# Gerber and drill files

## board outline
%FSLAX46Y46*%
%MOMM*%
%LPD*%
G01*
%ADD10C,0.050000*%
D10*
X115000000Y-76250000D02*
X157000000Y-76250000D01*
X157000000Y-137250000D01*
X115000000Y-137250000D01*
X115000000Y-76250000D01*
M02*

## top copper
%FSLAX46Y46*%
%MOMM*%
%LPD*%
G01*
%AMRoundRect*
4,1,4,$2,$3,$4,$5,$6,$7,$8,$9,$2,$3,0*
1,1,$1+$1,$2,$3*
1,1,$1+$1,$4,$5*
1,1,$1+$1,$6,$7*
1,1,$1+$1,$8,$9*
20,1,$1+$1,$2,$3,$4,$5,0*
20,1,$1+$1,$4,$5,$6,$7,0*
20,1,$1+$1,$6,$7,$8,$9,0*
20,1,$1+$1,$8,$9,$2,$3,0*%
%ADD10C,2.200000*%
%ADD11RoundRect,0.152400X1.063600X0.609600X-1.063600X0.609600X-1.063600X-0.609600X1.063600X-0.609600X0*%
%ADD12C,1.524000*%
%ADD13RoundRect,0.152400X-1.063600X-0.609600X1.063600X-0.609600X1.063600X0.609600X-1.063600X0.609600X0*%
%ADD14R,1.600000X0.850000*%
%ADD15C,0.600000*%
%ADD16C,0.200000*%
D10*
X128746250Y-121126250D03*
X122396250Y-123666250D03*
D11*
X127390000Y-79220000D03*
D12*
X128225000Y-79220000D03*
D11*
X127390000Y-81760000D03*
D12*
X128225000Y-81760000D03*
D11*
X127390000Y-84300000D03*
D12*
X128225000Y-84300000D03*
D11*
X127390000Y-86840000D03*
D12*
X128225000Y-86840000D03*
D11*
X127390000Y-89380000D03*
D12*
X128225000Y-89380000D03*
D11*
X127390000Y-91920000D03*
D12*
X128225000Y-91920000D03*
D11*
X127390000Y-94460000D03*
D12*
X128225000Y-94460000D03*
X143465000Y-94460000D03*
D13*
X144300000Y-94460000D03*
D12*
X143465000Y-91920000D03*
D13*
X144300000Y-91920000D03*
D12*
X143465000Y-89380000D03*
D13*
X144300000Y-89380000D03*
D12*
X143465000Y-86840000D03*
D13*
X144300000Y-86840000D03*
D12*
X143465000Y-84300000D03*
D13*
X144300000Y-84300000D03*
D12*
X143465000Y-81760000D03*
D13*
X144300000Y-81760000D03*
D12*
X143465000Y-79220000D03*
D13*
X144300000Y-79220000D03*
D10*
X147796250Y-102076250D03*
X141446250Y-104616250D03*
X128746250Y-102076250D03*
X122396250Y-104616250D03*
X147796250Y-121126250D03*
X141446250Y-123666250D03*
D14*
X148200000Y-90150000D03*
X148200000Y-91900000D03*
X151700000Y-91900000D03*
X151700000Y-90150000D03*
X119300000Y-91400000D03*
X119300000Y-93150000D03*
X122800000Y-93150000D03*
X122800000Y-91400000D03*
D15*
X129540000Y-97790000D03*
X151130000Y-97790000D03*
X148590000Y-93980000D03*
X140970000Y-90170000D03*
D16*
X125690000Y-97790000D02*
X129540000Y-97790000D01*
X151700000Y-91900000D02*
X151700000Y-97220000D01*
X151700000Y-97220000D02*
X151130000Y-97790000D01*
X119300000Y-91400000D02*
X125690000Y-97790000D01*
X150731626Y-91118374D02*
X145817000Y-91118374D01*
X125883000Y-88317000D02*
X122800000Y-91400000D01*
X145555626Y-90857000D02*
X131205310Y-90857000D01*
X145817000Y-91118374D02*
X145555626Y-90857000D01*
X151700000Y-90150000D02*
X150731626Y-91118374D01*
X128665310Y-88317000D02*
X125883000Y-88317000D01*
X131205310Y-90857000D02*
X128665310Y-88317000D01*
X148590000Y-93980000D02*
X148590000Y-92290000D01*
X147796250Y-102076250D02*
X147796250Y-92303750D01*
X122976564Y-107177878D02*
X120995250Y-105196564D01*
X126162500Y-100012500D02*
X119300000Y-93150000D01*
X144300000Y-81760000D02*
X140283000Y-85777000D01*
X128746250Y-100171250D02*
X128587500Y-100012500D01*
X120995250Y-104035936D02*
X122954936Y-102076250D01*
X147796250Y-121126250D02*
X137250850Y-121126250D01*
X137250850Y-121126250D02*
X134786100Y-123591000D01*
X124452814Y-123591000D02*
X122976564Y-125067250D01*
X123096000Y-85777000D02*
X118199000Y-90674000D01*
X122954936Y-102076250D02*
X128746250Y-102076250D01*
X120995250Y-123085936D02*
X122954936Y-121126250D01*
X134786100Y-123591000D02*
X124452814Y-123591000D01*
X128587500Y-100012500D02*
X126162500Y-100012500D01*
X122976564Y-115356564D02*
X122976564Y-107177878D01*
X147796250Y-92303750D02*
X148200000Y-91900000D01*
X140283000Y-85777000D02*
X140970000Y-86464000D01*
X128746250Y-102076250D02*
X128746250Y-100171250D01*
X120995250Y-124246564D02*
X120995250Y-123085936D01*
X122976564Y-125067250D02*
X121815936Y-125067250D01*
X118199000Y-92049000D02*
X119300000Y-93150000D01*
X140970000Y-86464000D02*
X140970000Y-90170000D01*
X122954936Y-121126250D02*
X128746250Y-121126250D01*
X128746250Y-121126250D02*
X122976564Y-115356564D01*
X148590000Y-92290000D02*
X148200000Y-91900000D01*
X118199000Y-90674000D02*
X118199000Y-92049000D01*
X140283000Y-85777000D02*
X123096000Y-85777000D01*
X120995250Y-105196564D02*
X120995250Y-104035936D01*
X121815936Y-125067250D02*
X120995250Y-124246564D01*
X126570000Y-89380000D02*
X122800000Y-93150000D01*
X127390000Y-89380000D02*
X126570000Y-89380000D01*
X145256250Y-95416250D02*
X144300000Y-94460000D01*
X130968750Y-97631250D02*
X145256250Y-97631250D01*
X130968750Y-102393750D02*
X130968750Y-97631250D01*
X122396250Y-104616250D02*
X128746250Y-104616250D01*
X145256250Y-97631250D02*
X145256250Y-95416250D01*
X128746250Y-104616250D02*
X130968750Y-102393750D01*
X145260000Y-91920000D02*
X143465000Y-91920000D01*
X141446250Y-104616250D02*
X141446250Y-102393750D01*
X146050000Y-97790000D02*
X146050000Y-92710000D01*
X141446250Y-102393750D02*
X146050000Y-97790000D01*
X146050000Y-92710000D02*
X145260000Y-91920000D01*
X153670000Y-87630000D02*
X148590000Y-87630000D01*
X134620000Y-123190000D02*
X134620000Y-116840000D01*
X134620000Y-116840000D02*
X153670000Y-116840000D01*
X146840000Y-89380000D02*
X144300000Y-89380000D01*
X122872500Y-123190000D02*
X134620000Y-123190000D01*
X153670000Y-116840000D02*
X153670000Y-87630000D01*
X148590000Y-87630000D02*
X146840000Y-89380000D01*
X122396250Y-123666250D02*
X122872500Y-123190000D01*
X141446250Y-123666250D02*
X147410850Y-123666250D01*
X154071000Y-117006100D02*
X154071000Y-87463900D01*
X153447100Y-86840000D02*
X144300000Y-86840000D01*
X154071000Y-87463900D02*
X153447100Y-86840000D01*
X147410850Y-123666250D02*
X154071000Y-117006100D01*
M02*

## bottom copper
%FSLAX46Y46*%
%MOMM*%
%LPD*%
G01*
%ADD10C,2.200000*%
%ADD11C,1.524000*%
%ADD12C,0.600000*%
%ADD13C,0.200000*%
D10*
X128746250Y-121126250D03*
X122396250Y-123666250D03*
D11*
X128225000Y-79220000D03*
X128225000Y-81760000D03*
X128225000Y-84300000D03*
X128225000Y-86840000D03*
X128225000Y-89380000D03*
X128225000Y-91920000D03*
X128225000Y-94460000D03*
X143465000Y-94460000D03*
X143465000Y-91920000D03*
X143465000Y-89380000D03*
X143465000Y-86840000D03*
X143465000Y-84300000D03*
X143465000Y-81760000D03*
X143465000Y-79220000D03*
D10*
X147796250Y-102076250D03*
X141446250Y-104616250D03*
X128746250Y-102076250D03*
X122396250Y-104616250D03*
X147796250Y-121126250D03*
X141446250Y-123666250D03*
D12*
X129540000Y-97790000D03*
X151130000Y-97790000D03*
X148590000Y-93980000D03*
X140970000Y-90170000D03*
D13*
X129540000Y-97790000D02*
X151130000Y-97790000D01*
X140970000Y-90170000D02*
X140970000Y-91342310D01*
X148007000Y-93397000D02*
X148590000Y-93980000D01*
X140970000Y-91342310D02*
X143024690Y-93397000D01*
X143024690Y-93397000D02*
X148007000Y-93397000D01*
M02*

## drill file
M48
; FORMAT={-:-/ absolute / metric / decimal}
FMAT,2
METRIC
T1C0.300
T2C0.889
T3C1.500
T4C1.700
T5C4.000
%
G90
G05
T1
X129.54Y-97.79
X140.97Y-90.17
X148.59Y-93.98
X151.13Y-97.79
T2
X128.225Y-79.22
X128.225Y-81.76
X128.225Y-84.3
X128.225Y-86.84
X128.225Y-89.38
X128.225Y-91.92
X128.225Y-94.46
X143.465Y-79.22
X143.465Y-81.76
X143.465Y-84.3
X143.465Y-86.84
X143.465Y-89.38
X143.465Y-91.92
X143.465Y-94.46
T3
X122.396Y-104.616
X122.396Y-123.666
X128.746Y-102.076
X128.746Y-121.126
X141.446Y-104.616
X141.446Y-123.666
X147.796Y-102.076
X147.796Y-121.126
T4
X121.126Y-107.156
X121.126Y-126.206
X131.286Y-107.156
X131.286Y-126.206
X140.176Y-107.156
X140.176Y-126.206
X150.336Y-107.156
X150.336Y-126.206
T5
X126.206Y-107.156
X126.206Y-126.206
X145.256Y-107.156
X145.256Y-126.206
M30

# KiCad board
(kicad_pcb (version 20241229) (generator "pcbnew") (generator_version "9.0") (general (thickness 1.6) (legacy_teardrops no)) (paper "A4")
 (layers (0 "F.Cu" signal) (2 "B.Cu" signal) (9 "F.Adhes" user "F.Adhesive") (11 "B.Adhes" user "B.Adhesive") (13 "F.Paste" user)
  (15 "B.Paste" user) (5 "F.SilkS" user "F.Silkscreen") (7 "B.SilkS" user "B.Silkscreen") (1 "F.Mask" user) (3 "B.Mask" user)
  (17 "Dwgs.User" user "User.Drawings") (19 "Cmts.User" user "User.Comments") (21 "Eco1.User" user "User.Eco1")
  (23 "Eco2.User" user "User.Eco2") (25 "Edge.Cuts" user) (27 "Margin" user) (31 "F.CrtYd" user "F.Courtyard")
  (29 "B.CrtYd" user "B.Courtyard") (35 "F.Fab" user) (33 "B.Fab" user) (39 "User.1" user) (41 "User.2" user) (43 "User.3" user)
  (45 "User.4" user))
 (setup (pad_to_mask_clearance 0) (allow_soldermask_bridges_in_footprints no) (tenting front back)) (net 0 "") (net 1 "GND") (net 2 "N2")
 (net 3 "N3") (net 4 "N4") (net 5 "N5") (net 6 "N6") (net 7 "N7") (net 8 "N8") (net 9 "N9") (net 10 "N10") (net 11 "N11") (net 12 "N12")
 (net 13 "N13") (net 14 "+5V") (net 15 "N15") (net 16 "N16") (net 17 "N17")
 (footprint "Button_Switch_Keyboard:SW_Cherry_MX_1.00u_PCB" (layer "F.Cu") (at 128.74625 121.12625)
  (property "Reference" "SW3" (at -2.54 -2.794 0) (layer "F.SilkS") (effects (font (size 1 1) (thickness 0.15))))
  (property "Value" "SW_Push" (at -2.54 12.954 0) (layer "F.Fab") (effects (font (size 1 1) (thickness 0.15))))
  (pad "" np_thru_hole circle (at -7.62 5.08) (size 1.7 1.7) (drill 1.7) (layers "*.Cu" "*.Mask"))
  (pad "" np_thru_hole circle (at -2.54 5.08) (size 4 4) (drill 4) (layers "*.Cu" "*.Mask"))
  (pad "" np_thru_hole circle (at 2.54 5.08) (size 1.7 1.7) (drill 1.7) (layers "*.Cu" "*.Mask"))
  (pad "1" thru_hole circle (at 0 0) (size 2.2 2.2) (drill 1.5) (layers "*.Cu" "*.Mask") (remove_unused_layers no) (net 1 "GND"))
  (pad "2" thru_hole circle (at -6.35 2.54) (size 2.2 2.2) (drill 1.5) (layers "*.Cu" "*.Mask") (remove_unused_layers no) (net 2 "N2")))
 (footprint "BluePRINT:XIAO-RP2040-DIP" (layer "F.Cu") (at 135.845 86.84)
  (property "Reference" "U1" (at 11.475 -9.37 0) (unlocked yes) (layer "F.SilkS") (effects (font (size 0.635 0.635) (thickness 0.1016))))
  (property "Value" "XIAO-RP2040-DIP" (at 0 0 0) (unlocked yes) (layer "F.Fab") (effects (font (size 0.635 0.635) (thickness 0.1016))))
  (pad "1" smd roundrect (at -8.455 -7.62 180) (size 2.432 1.524) (layers "F.Cu" "F.Mask") (roundrect_rratio 0.1) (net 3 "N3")
   (thermal_bridge_angle 45))
  (pad "1" thru_hole circle (at -7.62 -7.62 180) (size 1.524 1.524) (drill 0.889) (layers "*.Cu" "*.Mask") (remove_unused_layers no)
   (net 3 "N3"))
  (pad "2" smd roundrect (at -8.455 -5.08 180) (size 2.432 1.524) (layers "F.Cu" "F.Mask") (roundrect_rratio 0.1) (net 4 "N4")
   (thermal_bridge_angle 45))
  (pad "2" thru_hole circle (at -7.62 -5.08 180) (size 1.524 1.524) (drill 0.889) (layers "*.Cu" "*.Mask") (remove_unused_layers no)
   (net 4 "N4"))
  (pad "3" smd roundrect (at -8.455 -2.54 180) (size 2.432 1.524) (layers "F.Cu" "F.Mask") (roundrect_rratio 0.1) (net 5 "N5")
   (thermal_bridge_angle 45))
  (pad "3" thru_hole circle (at -7.62 -2.54 180) (size 1.524 1.524) (drill 0.889) (layers "*.Cu" "*.Mask") (remove_unused_layers no)
   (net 5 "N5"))
  (pad "4" smd roundrect (at -8.455 0 180) (size 2.432 1.524) (layers "F.Cu" "F.Mask") (roundrect_rratio 0.1) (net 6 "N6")
   (thermal_bridge_angle 45))
  (pad "4" thru_hole circle (at -7.62 0 180) (size 1.524 1.524) (drill 0.889) (layers "*.Cu" "*.Mask") (remove_unused_layers no)
   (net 6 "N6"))
  (pad "5" smd roundrect (at -8.455 2.54 180) (size 2.432 1.524) (layers "F.Cu" "F.Mask") (roundrect_rratio 0.1) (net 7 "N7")
   (thermal_bridge_angle 45))
  (pad "5" thru_hole circle (at -7.62 2.54 180) (size 1.524 1.524) (drill 0.889) (layers "*.Cu" "*.Mask") (remove_unused_layers no)
   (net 7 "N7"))
  (pad "6" smd roundrect (at -8.455 5.08 180) (size 2.432 1.524) (layers "F.Cu" "F.Mask") (roundrect_rratio 0.1) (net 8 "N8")
   (thermal_bridge_angle 45))
  (pad "6" thru_hole circle (at -7.62 5.08 180) (size 1.524 1.524) (drill 0.889) (layers "*.Cu" "*.Mask") (remove_unused_layers no)
   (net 8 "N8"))
  (pad "7" smd roundrect (at -8.455 7.62 180) (size 2.432 1.524) (layers "F.Cu" "F.Mask") (roundrect_rratio 0.1) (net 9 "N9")
   (thermal_bridge_angle 45))
  (pad "7" thru_hole circle (at -7.62 7.62 180) (size 1.524 1.524) (drill 0.889) (layers "*.Cu" "*.Mask") (remove_unused_layers no)
   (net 9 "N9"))
  (pad "8" thru_hole circle (at 7.62 7.62) (size 1.524 1.524) (drill 0.889) (layers "*.Cu" "*.Mask") (remove_unused_layers no)
   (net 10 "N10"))
  (pad "8" smd roundrect (at 8.455 7.62) (size 2.432 1.524) (layers "F.Cu" "F.Mask") (roundrect_rratio 0.1) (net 10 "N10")
   (thermal_bridge_angle 45))
  (pad "9" thru_hole circle (at 7.62 5.08) (size 1.524 1.524) (drill 0.889) (layers "*.Cu" "*.Mask") (remove_unused_layers no)
   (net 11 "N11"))
  (pad "9" smd roundrect (at 8.455 5.08) (size 2.432 1.524) (layers "F.Cu" "F.Mask") (roundrect_rratio 0.1) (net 11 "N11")
   (thermal_bridge_angle 45))
  (pad "10" thru_hole circle (at 7.62 2.54) (size 1.524 1.524) (drill 0.889) (layers "*.Cu" "*.Mask") (remove_unused_layers no) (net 2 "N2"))
  (pad "10" smd roundrect (at 8.455 2.54) (size 2.432 1.524) (layers "F.Cu" "F.Mask") (roundrect_rratio 0.1) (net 2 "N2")
   (thermal_bridge_angle 45))
  (pad "11" thru_hole circle (at 7.62 0) (size 1.524 1.524) (drill 0.889) (layers "*.Cu" "*.Mask") (remove_unused_layers no) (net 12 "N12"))
  (pad "11" smd roundrect (at 8.455 0) (size 2.432 1.524) (layers "F.Cu" "F.Mask") (roundrect_rratio 0.1) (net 12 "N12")
   (thermal_bridge_angle 45))
  (pad "12" thru_hole circle (at 7.62 -2.54) (size 1.524 1.524) (drill 0.889) (layers "*.Cu" "*.Mask") (remove_unused_layers no)
   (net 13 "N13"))
  (pad "12" smd roundrect (at 8.455 -2.54) (size 2.432 1.524) (layers "F.Cu" "F.Mask") (roundrect_rratio 0.1) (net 13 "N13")
   (thermal_bridge_angle 45))
  (pad "13" thru_hole circle (at 7.62 -5.08) (size 1.524 1.524) (drill 0.889) (layers "*.Cu" "*.Mask") (remove_unused_layers no)
   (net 1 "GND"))
  (pad "13" smd roundrect (at 8.455 -5.08) (size 2.432 1.524) (layers "F.Cu" "F.Mask") (roundrect_rratio 0.1) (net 1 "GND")
   (thermal_bridge_angle 45))
  (pad "14" thru_hole circle (at 7.62 -7.62) (size 1.524 1.524) (drill 0.889) (layers "*.Cu" "*.Mask") (remove_unused_layers no)
   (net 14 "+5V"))
  (pad "14" smd roundrect (at 8.455 -7.62) (size 2.432 1.524) (layers "F.Cu" "F.Mask") (roundrect_rratio 0.1) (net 14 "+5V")
   (thermal_bridge_angle 45)))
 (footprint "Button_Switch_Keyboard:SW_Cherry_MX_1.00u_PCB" (layer "F.Cu") (at 147.79625 102.07625)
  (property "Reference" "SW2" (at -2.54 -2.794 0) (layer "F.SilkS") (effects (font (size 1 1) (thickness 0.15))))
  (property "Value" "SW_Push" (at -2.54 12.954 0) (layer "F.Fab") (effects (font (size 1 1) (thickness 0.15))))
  (pad "" np_thru_hole circle (at -7.62 5.08) (size 1.7 1.7) (drill 1.7) (layers "*.Cu" "*.Mask"))
  (pad "" np_thru_hole circle (at -2.54 5.08) (size 4 4) (drill 4) (layers "*.Cu" "*.Mask"))
  (pad "" np_thru_hole circle (at 2.54 5.08) (size 1.7 1.7) (drill 1.7) (layers "*.Cu" "*.Mask"))
  (pad "1" thru_hole circle (at 0 0) (size 2.2 2.2) (drill 1.5) (layers "*.Cu" "*.Mask") (remove_unused_layers no) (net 1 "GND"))
  (pad "2" thru_hole circle (at -6.35 2.54) (size 2.2 2.2) (drill 1.5) (layers "*.Cu" "*.Mask") (remove_unused_layers no) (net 11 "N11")))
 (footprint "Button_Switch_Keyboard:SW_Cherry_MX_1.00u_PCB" (layer "F.Cu") (at 128.74625 102.07625)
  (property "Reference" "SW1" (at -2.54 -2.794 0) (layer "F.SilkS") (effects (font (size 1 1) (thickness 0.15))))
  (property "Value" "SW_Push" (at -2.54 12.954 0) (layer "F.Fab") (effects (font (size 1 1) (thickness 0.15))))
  (pad "" np_thru_hole circle (at -7.62 5.08) (size 1.7 1.7) (drill 1.7) (layers "*.Cu" "*.Mask"))
  (pad "" np_thru_hole circle (at -2.54 5.08) (size 4 4) (drill 4) (layers "*.Cu" "*.Mask"))
  (pad "" np_thru_hole circle (at 2.54 5.08) (size 1.7 1.7) (drill 1.7) (layers "*.Cu" "*.Mask"))
  (pad "1" thru_hole circle (at 0 0) (size 2.2 2.2) (drill 1.5) (layers "*.Cu" "*.Mask") (remove_unused_layers no) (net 1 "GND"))
  (pad "2" thru_hole circle (at -6.35 2.54) (size 2.2 2.2) (drill 1.5) (layers "*.Cu" "*.Mask") (remove_unused_layers no) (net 10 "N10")))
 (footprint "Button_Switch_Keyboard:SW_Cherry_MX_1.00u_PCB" (layer "F.Cu") (at 147.79625 121.12625)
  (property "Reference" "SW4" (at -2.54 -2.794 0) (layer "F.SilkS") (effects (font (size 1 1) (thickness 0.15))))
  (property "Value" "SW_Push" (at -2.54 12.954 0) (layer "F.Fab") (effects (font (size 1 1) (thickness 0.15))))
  (pad "" np_thru_hole circle (at -7.62 5.08) (size 1.7 1.7) (drill 1.7) (layers "*.Cu" "*.Mask"))
  (pad "" np_thru_hole circle (at -2.54 5.08) (size 4 4) (drill 4) (layers "*.Cu" "*.Mask"))
  (pad "" np_thru_hole circle (at 2.54 5.08) (size 1.7 1.7) (drill 1.7) (layers "*.Cu" "*.Mask"))
  (pad "1" thru_hole circle (at 0 0) (size 2.2 2.2) (drill 1.5) (layers "*.Cu" "*.Mask") (remove_unused_layers no) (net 1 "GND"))
  (pad "2" thru_hole circle (at -6.35 2.54) (size 2.2 2.2) (drill 1.5) (layers "*.Cu" "*.Mask") (remove_unused_layers no) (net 12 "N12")))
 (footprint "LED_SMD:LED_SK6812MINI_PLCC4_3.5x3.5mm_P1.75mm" (layer "F.Cu") (at 149.95 91.025)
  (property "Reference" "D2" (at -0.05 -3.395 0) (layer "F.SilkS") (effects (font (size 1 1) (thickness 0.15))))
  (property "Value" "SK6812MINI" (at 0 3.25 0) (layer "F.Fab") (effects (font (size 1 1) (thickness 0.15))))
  (pad "1" smd rect (at -1.75 -0.875) (size 1.6 0.85) (layers "F.Cu" "F.Mask" "F.Paste") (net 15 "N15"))
  (pad "2" smd rect (at -1.75 0.875) (size 1.6 0.85) (layers "F.Cu" "F.Mask" "F.Paste") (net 1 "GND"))
  (pad "3" smd rect (at 1.75 0.875) (size 1.6 0.85) (layers "F.Cu" "F.Mask" "F.Paste") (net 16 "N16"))
  (pad "4" smd rect (at 1.75 -0.875) (size 1.6 0.85) (layers "F.Cu" "F.Mask" "F.Paste") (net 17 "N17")))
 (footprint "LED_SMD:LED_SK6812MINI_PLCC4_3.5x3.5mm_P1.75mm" (layer "F.Cu") (at 121.05 92.275)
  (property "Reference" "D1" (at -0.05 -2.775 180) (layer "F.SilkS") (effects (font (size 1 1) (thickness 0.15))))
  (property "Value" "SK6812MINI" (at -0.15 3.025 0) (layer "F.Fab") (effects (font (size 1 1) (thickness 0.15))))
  (pad "1" smd rect (at -1.75 -0.875) (size 1.6 0.85) (layers "F.Cu" "F.Mask" "F.Paste") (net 16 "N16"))
  (pad "2" smd rect (at -1.75 0.875) (size 1.6 0.85) (layers "F.Cu" "F.Mask" "F.Paste") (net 1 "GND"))
  (pad "3" smd rect (at 1.75 0.875) (size 1.6 0.85) (layers "F.Cu" "F.Mask" "F.Paste") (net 7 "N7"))
  (pad "4" smd rect (at 1.75 -0.875) (size 1.6 0.85) (layers "F.Cu" "F.Mask" "F.Paste") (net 17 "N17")))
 (gr_rect (start 115 76.25) (end 157 137.25) (stroke (width 0.05) (type default)) (fill no) (layer "Edge.Cuts"))
 (segment (start 125.69 97.79) (end 129.54 97.79) (width 0.2) (layer "F.Cu") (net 16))
 (segment (start 151.7 91.9) (end 151.7 97.22) (width 0.2) (layer "F.Cu") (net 16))
 (segment (start 151.7 97.22) (end 151.13 97.79) (width 0.2) (layer "F.Cu") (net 16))
 (segment (start 119.3 91.4) (end 125.69 97.79) (width 0.2) (layer "F.Cu") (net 16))
 (via (at 129.54 97.79) (size 0.6) (drill 0.3) (layers "F.Cu" "B.Cu") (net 16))
 (via (at 151.13 97.79) (size 0.6) (drill 0.3) (layers "F.Cu" "B.Cu") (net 16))
 (segment (start 129.54 97.79) (end 151.13 97.79) (width 0.2) (layer "B.Cu") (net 16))
 (segment (start 150.731626 91.118374) (end 145.817 91.118374) (width 0.2) (layer "F.Cu") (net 17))
 (segment (start 125.883 88.317) (end 122.8 91.4) (width 0.2) (layer "F.Cu") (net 17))
 (segment (start 145.555626 90.857) (end 131.20531 90.857) (width 0.2) (layer "F.Cu") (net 17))
 (segment (start 145.817 91.118374) (end 145.555626 90.857) (width 0.2) (layer "F.Cu") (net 17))
 (segment (start 151.7 90.15) (end 150.731626 91.118374) (width 0.2) (layer "F.Cu") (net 17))
 (segment (start 128.66531 88.317) (end 125.883 88.317) (width 0.2) (layer "F.Cu") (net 17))
 (segment (start 131.20531 90.857) (end 128.66531 88.317) (width 0.2) (layer "F.Cu") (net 17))
 (segment (start 148.59 93.98) (end 148.59 92.29) (width 0.2) (layer "F.Cu") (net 1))
 (segment (start 147.79625 102.07625) (end 147.79625 92.30375) (width 0.2) (layer "F.Cu") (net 1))
 (segment (start 122.976564 107.177878) (end 120.99525 105.196564) (width 0.2) (layer "F.Cu") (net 1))
 (segment (start 126.1625 100.0125) (end 119.3 93.15) (width 0.2) (layer "F.Cu") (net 1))
 (segment (start 144.3 81.76) (end 140.283 85.777) (width 0.2) (layer "F.Cu") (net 1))
 (segment (start 128.74625 100.17125) (end 128.5875 100.0125) (width 0.2) (layer "F.Cu") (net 1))
 (segment (start 120.99525 104.035936) (end 122.954936 102.07625) (width 0.2) (layer "F.Cu") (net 1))
 (segment (start 147.79625 121.12625) (end 137.25085 121.12625) (width 0.2) (layer "F.Cu") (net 1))
 (segment (start 137.25085 121.12625) (end 134.7861 123.591) (width 0.2) (layer "F.Cu") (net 1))
 (segment (start 124.452814 123.591) (end 122.976564 125.06725) (width 0.2) (layer "F.Cu") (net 1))
 (segment (start 123.096 85.777) (end 118.199 90.674) (width 0.2) (layer "F.Cu") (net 1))
 (segment (start 122.954936 102.07625) (end 128.74625 102.07625) (width 0.2) (layer "F.Cu") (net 1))
 (segment (start 120.99525 123.085936) (end 122.954936 121.12625) (width 0.2) (layer "F.Cu") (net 1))
 (segment (start 134.7861 123.591) (end 124.452814 123.591) (width 0.2) (layer "F.Cu") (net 1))
 (segment (start 128.5875 100.0125) (end 126.1625 100.0125) (width 0.2) (layer "F.Cu") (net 1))
 (segment (start 122.976564 115.356564) (end 122.976564 107.177878) (width 0.2) (layer "F.Cu") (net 1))
 (segment (start 147.79625 92.30375) (end 148.2 91.9) (width 0.2) (layer "F.Cu") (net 1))
 (segment (start 140.283 85.777) (end 140.97 86.464) (width 0.2) (layer "F.Cu") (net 1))
 (segment (start 128.74625 102.07625) (end 128.74625 100.17125) (width 0.2) (layer "F.Cu") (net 1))
 (segment (start 120.99525 124.246564) (end 120.99525 123.085936) (width 0.2) (layer "F.Cu") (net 1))
 (segment (start 122.976564 125.06725) (end 121.815936 125.06725) (width 0.2) (layer "F.Cu") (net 1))
 (segment (start 118.199 92.049) (end 119.3 93.15) (width 0.2) (layer "F.Cu") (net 1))
 (segment (start 140.97 86.464) (end 140.97 90.17) (width 0.2) (layer "F.Cu") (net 1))
 (segment (start 122.954936 121.12625) (end 128.74625 121.12625) (width 0.2) (layer "F.Cu") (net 1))
 (segment (start 128.74625 121.12625) (end 122.976564 115.356564) (width 0.2) (layer "F.Cu") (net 1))
 (segment (start 148.59 92.29) (end 148.2 91.9) (width 0.2) (layer "F.Cu") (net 1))
 (segment (start 118.199 90.674) (end 118.199 92.049) (width 0.2) (layer "F.Cu") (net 1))
 (segment (start 140.283 85.777) (end 123.096 85.777) (width 0.2) (layer "F.Cu") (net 1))
 (segment (start 120.99525 105.196564) (end 120.99525 104.035936) (width 0.2) (layer "F.Cu") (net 1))
 (segment (start 121.815936 125.06725) (end 120.99525 124.246564) (width 0.2) (layer "F.Cu") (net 1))
 (via (at 148.59 93.98) (size 0.6) (drill 0.3) (layers "F.Cu" "B.Cu") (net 1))
 (via (at 140.97 90.17) (size 0.6) (drill 0.3) (layers "F.Cu" "B.Cu") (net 1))
 (segment (start 140.97 90.17) (end 140.97 91.34231) (width 0.2) (layer "B.Cu") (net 1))
 (segment (start 148.007 93.397) (end 148.59 93.98) (width 0.2) (layer "B.Cu") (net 1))
 (segment (start 140.97 91.34231) (end 143.02469 93.397) (width 0.2) (layer "B.Cu") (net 1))
 (segment (start 143.02469 93.397) (end 148.007 93.397) (width 0.2) (layer "B.Cu") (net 1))
 (segment (start 126.57 89.38) (end 122.8 93.15) (width 0.2) (layer "F.Cu") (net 7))
 (segment (start 127.39 89.38) (end 126.57 89.38) (width 0.2) (layer "F.Cu") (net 7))
 (segment (start 145.25625 95.41625) (end 144.3 94.46) (width 0.2) (layer "F.Cu") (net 10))
 (segment (start 130.96875 97.63125) (end 145.25625 97.63125) (width 0.2) (layer "F.Cu") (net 10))
 (segment (start 130.96875 102.39375) (end 130.96875 97.63125) (width 0.2) (layer "F.Cu") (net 10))
 (segment (start 122.39625 104.61625) (end 128.74625 104.61625) (width 0.2) (layer "F.Cu") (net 10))
 (segment (start 145.25625 97.63125) (end 145.25625 95.41625) (width 0.2) (layer "F.Cu") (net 10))
 (segment (start 128.74625 104.61625) (end 130.96875 102.39375) (width 0.2) (layer "F.Cu") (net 10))
 (segment (start 145.26 91.92) (end 143.465 91.92) (width 0.2) (layer "F.Cu") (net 11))
 (segment (start 141.44625 104.61625) (end 141.44625 102.39375) (width 0.2) (layer "F.Cu") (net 11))
 (segment (start 146.05 97.79) (end 146.05 92.71) (width 0.2) (layer "F.Cu") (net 11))
 (segment (start 141.44625 102.39375) (end 146.05 97.79) (width 0.2) (layer "F.Cu") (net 11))
 (segment (start 146.05 92.71) (end 145.26 91.92) (width 0.2) (layer "F.Cu") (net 11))
 (segment (start 153.67 87.63) (end 148.59 87.63) (width 0.2) (layer "F.Cu") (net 2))
 (segment (start 134.62 123.19) (end 134.62 116.84) (width 0.2) (layer "F.Cu") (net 2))
 (segment (start 134.62 116.84) (end 153.67 116.84) (width 0.2) (layer "F.Cu") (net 2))
 (segment (start 146.84 89.38) (end 144.3 89.38) (width 0.2) (layer "F.Cu") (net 2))
 (segment (start 122.8725 123.19) (end 134.62 123.19) (width 0.2) (layer "F.Cu") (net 2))
 (segment (start 153.67 116.84) (end 153.67 87.63) (width 0.2) (layer "F.Cu") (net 2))
 (segment (start 148.59 87.63) (end 146.84 89.38) (width 0.2) (layer "F.Cu") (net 2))
 (segment (start 122.39625 123.66625) (end 122.8725 123.19) (width 0.2) (layer "F.Cu") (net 2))
 (segment (start 141.44625 123.66625) (end 147.41085 123.66625) (width 0.2) (layer "F.Cu") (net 12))
 (segment (start 154.071 117.0061) (end 154.071 87.4639) (width 0.2) (layer "F.Cu") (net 12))
 (segment (start 153.4471 86.84) (end 144.3 86.84) (width 0.2) (layer "F.Cu") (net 12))
 (segment (start 154.071 87.4639) (end 153.4471 86.84) (width 0.2) (layer "F.Cu") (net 12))
 (segment (start 147.41085 123.66625) (end 154.071 117.0061) (width 0.2) (layer "F.Cu") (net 12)))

